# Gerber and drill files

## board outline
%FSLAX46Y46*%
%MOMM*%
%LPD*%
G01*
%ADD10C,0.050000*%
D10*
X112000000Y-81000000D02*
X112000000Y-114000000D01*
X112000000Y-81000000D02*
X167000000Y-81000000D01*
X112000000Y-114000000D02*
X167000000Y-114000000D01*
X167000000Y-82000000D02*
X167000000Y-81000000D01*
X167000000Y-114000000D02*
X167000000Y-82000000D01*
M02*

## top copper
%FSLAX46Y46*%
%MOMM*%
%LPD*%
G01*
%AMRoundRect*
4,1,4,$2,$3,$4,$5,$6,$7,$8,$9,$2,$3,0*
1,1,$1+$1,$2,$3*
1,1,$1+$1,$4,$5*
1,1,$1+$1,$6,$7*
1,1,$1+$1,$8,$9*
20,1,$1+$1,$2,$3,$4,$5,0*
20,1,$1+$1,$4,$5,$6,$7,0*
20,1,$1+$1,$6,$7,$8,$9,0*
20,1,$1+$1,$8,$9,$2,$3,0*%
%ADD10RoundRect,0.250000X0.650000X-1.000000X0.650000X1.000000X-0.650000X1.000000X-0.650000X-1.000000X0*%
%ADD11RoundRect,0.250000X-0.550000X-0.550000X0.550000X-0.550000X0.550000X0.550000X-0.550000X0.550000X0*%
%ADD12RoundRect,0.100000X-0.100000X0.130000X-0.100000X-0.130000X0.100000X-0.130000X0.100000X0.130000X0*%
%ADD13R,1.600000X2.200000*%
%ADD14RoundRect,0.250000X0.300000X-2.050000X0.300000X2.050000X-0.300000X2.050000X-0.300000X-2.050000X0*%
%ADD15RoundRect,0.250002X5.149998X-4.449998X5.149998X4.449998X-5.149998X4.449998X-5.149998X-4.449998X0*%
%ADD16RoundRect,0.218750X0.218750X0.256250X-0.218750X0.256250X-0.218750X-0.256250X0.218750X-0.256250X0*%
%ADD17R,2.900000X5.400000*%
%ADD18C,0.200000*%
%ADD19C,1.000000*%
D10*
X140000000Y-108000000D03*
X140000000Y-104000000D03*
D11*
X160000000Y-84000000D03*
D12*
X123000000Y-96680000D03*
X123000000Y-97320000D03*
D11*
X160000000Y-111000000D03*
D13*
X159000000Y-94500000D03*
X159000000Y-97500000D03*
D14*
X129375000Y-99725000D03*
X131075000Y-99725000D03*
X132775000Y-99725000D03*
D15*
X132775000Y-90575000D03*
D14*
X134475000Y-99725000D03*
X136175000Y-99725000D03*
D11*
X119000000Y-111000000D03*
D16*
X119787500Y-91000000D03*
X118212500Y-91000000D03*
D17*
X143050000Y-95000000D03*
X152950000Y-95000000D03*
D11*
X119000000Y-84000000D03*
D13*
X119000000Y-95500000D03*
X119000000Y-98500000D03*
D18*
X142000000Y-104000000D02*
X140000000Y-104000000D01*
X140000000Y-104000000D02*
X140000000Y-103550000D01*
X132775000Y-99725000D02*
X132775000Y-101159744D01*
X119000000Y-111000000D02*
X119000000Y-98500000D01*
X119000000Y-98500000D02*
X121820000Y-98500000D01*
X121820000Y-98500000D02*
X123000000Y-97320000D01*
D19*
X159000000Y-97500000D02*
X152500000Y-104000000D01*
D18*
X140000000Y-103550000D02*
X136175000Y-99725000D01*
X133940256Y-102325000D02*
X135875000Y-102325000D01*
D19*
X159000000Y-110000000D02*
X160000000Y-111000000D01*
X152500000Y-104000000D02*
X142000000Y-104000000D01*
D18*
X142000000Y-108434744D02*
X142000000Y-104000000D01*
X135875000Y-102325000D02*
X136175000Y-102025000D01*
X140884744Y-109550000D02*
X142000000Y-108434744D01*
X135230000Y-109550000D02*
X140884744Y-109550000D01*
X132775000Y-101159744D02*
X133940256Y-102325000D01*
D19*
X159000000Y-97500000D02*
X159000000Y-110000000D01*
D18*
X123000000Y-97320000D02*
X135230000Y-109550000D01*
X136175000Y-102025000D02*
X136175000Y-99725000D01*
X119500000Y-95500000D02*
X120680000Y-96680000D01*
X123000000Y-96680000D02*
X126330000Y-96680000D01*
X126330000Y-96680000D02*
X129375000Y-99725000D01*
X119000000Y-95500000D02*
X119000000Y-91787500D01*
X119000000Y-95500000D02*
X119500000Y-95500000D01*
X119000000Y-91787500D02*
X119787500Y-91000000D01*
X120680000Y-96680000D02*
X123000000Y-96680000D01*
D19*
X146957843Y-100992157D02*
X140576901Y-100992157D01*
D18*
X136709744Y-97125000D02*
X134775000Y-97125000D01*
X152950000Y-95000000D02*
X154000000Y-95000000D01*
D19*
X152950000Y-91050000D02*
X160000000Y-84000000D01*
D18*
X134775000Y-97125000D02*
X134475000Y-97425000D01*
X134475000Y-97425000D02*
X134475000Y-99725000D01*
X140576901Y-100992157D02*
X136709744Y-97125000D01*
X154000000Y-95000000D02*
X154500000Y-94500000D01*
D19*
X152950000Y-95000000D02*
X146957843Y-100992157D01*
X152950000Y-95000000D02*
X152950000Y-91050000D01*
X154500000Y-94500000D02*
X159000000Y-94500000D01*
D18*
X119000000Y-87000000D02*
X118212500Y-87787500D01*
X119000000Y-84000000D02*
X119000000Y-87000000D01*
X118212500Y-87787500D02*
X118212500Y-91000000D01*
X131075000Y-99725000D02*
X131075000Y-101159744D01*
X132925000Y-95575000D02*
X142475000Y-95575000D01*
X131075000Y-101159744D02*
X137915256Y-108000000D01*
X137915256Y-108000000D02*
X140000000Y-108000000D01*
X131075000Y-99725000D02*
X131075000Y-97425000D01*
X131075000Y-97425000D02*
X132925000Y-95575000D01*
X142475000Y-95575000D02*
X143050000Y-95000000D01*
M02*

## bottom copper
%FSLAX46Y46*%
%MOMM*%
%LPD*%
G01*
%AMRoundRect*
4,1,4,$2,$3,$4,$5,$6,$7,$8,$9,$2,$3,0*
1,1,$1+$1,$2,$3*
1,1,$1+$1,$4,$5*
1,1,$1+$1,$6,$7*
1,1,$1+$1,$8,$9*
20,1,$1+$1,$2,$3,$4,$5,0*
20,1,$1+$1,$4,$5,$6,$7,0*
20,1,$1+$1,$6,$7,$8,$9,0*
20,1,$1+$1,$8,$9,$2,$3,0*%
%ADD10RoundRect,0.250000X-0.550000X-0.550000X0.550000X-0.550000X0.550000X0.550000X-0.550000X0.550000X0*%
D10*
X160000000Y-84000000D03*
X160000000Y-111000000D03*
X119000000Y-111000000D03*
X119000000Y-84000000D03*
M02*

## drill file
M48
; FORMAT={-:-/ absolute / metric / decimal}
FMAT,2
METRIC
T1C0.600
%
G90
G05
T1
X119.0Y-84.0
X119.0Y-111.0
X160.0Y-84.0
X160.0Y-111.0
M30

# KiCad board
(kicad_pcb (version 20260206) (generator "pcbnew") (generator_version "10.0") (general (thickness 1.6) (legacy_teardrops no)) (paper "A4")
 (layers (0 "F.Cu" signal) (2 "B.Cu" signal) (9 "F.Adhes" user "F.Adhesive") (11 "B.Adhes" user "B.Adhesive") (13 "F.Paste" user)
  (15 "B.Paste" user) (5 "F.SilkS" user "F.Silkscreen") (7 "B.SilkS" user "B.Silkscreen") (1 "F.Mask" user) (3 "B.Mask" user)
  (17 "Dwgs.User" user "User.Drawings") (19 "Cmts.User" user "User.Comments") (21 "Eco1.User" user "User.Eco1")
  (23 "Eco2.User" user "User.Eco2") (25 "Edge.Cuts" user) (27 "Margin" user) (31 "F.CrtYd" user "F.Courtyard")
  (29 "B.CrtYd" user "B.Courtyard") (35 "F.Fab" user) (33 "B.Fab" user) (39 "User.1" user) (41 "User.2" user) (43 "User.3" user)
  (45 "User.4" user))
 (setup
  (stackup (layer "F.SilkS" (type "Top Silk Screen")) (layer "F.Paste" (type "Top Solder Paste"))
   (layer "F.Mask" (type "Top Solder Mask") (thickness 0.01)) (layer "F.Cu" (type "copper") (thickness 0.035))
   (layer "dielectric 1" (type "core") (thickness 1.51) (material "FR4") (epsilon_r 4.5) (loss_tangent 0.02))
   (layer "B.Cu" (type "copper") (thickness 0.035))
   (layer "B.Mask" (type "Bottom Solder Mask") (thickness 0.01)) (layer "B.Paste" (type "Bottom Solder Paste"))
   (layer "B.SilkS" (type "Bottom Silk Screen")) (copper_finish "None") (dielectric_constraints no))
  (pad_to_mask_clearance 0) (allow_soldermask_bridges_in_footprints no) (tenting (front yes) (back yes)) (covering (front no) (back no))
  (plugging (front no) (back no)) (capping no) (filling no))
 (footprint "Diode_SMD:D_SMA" (layer "F.Cu") (at 140 106 90)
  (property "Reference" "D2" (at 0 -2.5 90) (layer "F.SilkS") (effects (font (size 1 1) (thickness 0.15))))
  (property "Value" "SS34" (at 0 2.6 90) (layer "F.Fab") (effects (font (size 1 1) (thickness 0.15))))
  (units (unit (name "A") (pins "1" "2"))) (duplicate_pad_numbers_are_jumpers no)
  (pad "1" smd roundrect (at -2 0 90) (size 2.5 1.8) (layers "F.Cu" "F.Mask" "F.Paste") (roundrect_rratio 0.1388888889) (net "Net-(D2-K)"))
  (pad "2" smd roundrect (at 2 0 90) (size 2.5 1.8) (layers "F.Cu" "F.Mask" "F.Paste") (roundrect_rratio 0.1388888889) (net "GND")))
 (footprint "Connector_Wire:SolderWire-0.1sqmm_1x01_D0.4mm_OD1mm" (layer "F.Cu") (at 160 84)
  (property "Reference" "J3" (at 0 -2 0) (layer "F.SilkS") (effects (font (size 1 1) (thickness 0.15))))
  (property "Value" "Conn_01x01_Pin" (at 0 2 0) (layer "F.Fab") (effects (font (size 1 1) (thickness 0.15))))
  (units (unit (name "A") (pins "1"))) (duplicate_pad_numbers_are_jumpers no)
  (pad "1" thru_hole roundrect (at 0 0) (size 1.6 1.6) (drill 0.6) (layers "*.Cu" "*.Mask") (remove_unused_layers no)
   (roundrect_rratio 0.15625) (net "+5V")))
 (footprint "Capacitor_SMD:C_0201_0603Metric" (layer "F.Cu") (at 123 97 -90)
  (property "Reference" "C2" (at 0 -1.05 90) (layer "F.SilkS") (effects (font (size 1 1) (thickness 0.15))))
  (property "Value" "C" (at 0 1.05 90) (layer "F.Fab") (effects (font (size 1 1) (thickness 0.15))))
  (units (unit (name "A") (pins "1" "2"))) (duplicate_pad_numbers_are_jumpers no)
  (pad "" smd roundrect (at -0.345 0 270) (size 0.318 0.36) (layers "F.Paste") (roundrect_rratio 0.25))
  (pad "" smd roundrect (at 0.345 0 270) (size 0.318 0.36) (layers "F.Paste") (roundrect_rratio 0.25))
  (pad "1" smd roundrect (at -0.32 0 270) (size 0.46 0.4) (layers "F.Cu" "F.Mask") (roundrect_rratio 0.25) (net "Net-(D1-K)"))
  (pad "2" smd roundrect (at 0.32 0 270) (size 0.46 0.4) (layers "F.Cu" "F.Mask") (roundrect_rratio 0.25) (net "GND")))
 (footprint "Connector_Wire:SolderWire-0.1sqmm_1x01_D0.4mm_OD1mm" (layer "F.Cu") (at 160 111)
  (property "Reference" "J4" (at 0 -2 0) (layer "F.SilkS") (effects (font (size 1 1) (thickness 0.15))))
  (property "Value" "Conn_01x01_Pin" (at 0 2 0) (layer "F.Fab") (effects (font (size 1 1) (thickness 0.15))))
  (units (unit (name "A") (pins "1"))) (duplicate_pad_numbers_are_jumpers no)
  (pad "1" thru_hole roundrect (at 0 0) (size 1.6 1.6) (drill 0.6) (layers "*.Cu" "*.Mask") (remove_unused_layers no)
   (roundrect_rratio 0.15625) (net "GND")))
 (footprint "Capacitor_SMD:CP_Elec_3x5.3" (layer "F.Cu") (at 159 96 -90)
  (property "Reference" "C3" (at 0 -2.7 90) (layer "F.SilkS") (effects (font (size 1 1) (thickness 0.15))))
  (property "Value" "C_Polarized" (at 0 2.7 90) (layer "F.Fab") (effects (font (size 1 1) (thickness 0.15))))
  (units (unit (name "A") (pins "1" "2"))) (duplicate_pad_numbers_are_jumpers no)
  (pad "1" smd rect (at -1.5 0 270) (size 2.2 1.6) (layers "F.Cu" "F.Mask" "F.Paste") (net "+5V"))
  (pad "2" smd rect (at 1.5 0 270) (size 2.2 1.6) (layers "F.Cu" "F.Mask" "F.Paste") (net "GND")))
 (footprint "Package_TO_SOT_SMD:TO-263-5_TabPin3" (layer "F.Cu") (at 132.775 92.075 90)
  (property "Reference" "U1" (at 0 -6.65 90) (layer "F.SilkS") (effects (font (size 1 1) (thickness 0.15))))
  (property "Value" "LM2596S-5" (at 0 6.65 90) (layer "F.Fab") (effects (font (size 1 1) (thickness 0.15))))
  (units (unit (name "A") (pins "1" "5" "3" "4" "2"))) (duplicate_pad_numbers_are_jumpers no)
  (pad "" smd roundrect (at -0.925 -2.775 90) (size 4.55 5.25) (layers "F.Paste") (roundrect_rratio 0.054945))
  (pad "" smd roundrect (at -0.925 2.775 90) (size 4.55 5.25) (layers "F.Paste") (roundrect_rratio 0.054945))
  (pad "" smd roundrect (at 3.925 -2.775 90) (size 4.55 5.25) (layers "F.Paste") (roundrect_rratio 0.054945))
  (pad "" smd roundrect (at 3.925 2.775 90) (size 4.55 5.25) (layers "F.Paste") (roundrect_rratio 0.054945))
  (pad "1" smd roundrect (at -7.65 -3.4 90) (size 4.6 1.1) (layers "F.Cu" "F.Mask" "F.Paste") (roundrect_rratio 0.227273) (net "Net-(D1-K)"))
  (pad "2" smd roundrect (at -7.65 -1.7 90) (size 4.6 1.1) (layers "F.Cu" "F.Mask" "F.Paste") (roundrect_rratio 0.227273) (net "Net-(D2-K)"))
  (pad "3" smd roundrect (at -7.65 0 90) (size 4.6 1.1) (layers "F.Cu" "F.Mask" "F.Paste") (roundrect_rratio 0.227273) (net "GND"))
  (pad "3" smd roundrect (at 1.5 0 90) (size 9.4 10.8) (layers "F.Cu" "F.Mask") (roundrect_rratio 0.026596) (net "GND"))
  (pad "4" smd roundrect (at -7.65 1.7 90) (size 4.6 1.1) (layers "F.Cu" "F.Mask" "F.Paste") (roundrect_rratio 0.227273) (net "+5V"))
  (pad "5" smd roundrect (at -7.65 3.4 90) (size 4.6 1.1) (layers "F.Cu" "F.Mask" "F.Paste") (roundrect_rratio 0.227273) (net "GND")))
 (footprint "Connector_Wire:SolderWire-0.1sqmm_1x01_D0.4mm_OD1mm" (layer "F.Cu") (at 119 111)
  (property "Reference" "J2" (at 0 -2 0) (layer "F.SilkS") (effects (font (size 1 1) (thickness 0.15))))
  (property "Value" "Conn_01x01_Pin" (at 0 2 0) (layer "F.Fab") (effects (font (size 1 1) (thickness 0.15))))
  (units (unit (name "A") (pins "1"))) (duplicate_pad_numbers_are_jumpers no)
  (pad "1" thru_hole roundrect (at 0 0) (size 1.6 1.6) (drill 0.6) (layers "*.Cu" "*.Mask") (remove_unused_layers no)
   (roundrect_rratio 0.15625) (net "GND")))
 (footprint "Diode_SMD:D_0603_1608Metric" (layer "F.Cu") (at 119 91 180)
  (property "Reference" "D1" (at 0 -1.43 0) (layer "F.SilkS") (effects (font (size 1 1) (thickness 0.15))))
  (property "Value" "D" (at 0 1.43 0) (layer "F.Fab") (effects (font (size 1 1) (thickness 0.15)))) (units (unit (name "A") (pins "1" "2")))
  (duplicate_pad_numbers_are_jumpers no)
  (pad "1" smd roundrect (at -0.7875 0 180) (size 0.875 0.95) (layers "F.Cu" "F.Mask" "F.Paste") (roundrect_rratio 0.25) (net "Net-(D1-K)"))
  (pad "2" smd roundrect (at 0.7875 0 180) (size 0.875 0.95) (layers "F.Cu" "F.Mask" "F.Paste") (roundrect_rratio 0.25) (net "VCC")))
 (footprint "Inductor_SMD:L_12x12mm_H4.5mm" (layer "F.Cu") (at 148 95)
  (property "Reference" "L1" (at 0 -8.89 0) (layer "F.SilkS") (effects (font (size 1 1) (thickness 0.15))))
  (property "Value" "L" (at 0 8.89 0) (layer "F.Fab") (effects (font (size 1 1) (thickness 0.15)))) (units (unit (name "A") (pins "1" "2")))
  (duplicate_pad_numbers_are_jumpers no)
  (pad "1" smd rect (at -4.95 0) (size 2.9 5.4) (layers "F.Cu" "F.Mask" "F.Paste") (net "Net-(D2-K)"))
  (pad "2" smd rect (at 4.95 0) (size 2.9 5.4) (layers "F.Cu" "F.Mask" "F.Paste") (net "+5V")))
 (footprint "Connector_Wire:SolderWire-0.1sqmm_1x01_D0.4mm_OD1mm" (layer "F.Cu") (at 119 84)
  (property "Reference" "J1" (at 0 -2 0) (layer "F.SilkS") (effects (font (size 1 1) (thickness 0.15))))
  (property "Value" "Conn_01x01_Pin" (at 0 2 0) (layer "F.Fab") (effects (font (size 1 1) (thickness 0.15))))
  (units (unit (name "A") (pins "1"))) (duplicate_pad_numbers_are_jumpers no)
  (pad "1" thru_hole roundrect (at 0 0) (size 1.6 1.6) (drill 0.6) (layers "*.Cu" "*.Mask") (remove_unused_layers no)
   (roundrect_rratio 0.15625) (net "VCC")))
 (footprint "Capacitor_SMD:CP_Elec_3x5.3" (layer "F.Cu") (at 119 97 -90)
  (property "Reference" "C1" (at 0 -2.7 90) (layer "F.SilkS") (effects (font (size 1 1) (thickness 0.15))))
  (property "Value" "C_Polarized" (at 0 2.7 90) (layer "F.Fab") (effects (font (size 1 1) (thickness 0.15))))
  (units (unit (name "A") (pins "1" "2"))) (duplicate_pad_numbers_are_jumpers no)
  (pad "1" smd rect (at -1.5 0 270) (size 2.2 1.6) (layers "F.Cu" "F.Mask" "F.Paste") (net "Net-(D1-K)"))
  (pad "2" smd rect (at 1.5 0 270) (size 2.2 1.6) (layers "F.Cu" "F.Mask" "F.Paste") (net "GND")))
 (gr_line (start 112 81) (end 112 114) (stroke (width 0.05) (type default)) (layer "Edge.Cuts"))
 (gr_line (start 112 81) (end 167 81) (stroke (width 0.05) (type default)) (layer "Edge.Cuts"))
 (gr_line (start 112 114) (end 167 114) (stroke (width 0.05) (type default)) (layer "Edge.Cuts"))
 (gr_line (start 167 82) (end 167 81) (stroke (width 0.05) (type default)) (layer "Edge.Cuts"))
 (gr_line (start 167 114) (end 167 82) (stroke (width 0.05) (type default)) (layer "Edge.Cuts"))
 (segment (start 142 104) (end 140 104) (width 0.2) (layer "F.Cu") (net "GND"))
 (segment (start 140 104) (end 140 103.55) (width 0.2) (layer "F.Cu") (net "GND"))
 (segment (start 132.775 99.725) (end 132.775 101.159744) (width 0.2) (layer "F.Cu") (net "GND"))
 (segment (start 119 111) (end 119 98.5) (width 0.2) (layer "F.Cu") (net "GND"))
 (segment (start 119 98.5) (end 121.82 98.5) (width 0.2) (layer "F.Cu") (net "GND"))
 (segment (start 121.82 98.5) (end 123 97.32) (width 0.2) (layer "F.Cu") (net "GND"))
 (segment (start 159 97.5) (end 152.5 104) (width 1) (layer "F.Cu") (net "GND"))
 (segment (start 140 103.55) (end 136.175 99.725) (width 0.2) (layer "F.Cu") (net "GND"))
 (segment (start 133.940256 102.325) (end 135.875 102.325) (width 0.2) (layer "F.Cu") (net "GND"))
 (segment (start 159 110) (end 160 111) (width 1) (layer "F.Cu") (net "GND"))
 (segment (start 152.5 104) (end 142 104) (width 1) (layer "F.Cu") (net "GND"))
 (segment (start 142 108.434744) (end 142 104) (width 0.2) (layer "F.Cu") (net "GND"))
 (segment (start 135.875 102.325) (end 136.175 102.025) (width 0.2) (layer "F.Cu") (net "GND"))
 (segment (start 140.884744 109.55) (end 142 108.434744) (width 0.2) (layer "F.Cu") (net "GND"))
 (segment (start 135.23 109.55) (end 140.884744 109.55) (width 0.2) (layer "F.Cu") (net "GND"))
 (segment (start 132.775 101.159744) (end 133.940256 102.325) (width 0.2) (layer "F.Cu") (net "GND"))
 (segment (start 159 97.5) (end 159 110) (width 1) (layer "F.Cu") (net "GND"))
 (segment (start 123 97.32) (end 135.23 109.55) (width 0.2) (layer "F.Cu") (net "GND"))
 (segment (start 136.175 102.025) (end 136.175 99.725) (width 0.2) (layer "F.Cu") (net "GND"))
 (segment (start 119.5 95.5) (end 120.68 96.68) (width 0.2) (layer "F.Cu") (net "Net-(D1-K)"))
 (segment (start 123 96.68) (end 126.33 96.68) (width 0.2) (layer "F.Cu") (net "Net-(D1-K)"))
 (segment (start 126.33 96.68) (end 129.375 99.725) (width 0.2) (layer "F.Cu") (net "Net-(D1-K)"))
 (segment (start 119 95.5) (end 119 91.7875) (width 0.2) (layer "F.Cu") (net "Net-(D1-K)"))
 (segment (start 119 95.5) (end 119.5 95.5) (width 0.2) (layer "F.Cu") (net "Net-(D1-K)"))
 (segment (start 119 91.7875) (end 119.7875 91) (width 0.2) (layer "F.Cu") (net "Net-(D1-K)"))
 (segment (start 120.68 96.68) (end 123 96.68) (width 0.2) (layer "F.Cu") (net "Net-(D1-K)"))
 (segment (start 146.957843 100.992157) (end 140.576901 100.992157) (width 1) (layer "F.Cu") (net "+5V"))
 (segment (start 136.709744 97.125) (end 134.775 97.125) (width 0.2) (layer "F.Cu") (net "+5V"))
 (segment (start 152.95 95) (end 154 95) (width 0.2) (layer "F.Cu") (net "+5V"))
 (segment (start 152.95 91.05) (end 160 84) (width 1) (layer "F.Cu") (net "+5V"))
 (segment (start 134.775 97.125) (end 134.475 97.425) (width 0.2) (layer "F.Cu") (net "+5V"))
 (segment (start 134.475 97.425) (end 134.475 99.725) (width 0.2) (layer "F.Cu") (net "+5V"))
 (segment (start 140.576901 100.992157) (end 136.709744 97.125) (width 0.2) (layer "F.Cu") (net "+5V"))
 (segment (start 154 95) (end 154.5 94.5) (width 0.2) (layer "F.Cu") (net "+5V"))
 (segment (start 152.95 95) (end 146.957843 100.992157) (width 1) (layer "F.Cu") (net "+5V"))
 (segment (start 152.95 95) (end 152.95 91.05) (width 1) (layer "F.Cu") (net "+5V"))
 (segment (start 154.5 94.5) (end 159 94.5) (width 1) (layer "F.Cu") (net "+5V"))
 (segment (start 119 87) (end 118.2125 87.7875) (width 0.2) (layer "F.Cu") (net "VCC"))
 (segment (start 119 84) (end 119 87) (width 0.2) (layer "F.Cu") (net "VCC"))
 (segment (start 118.2125 87.7875) (end 118.2125 91) (width 0.2) (layer "F.Cu") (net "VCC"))
 (segment (start 131.075 99.725) (end 131.075 101.159744) (width 0.2) (layer "F.Cu") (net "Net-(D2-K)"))
 (segment (start 132.925 95.575) (end 142.475 95.575) (width 0.2) (layer "F.Cu") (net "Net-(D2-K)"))
 (segment (start 131.075 101.159744) (end 137.915256 108) (width 0.2) (layer "F.Cu") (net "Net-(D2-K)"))
 (segment (start 137.915256 108) (end 140 108) (width 0.2) (layer "F.Cu") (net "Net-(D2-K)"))
 (segment (start 131.075 99.725) (end 131.075 97.425) (width 0.2) (layer "F.Cu") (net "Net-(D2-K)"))
 (segment (start 131.075 97.425) (end 132.925 95.575) (width 0.2) (layer "F.Cu") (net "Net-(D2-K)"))
 (segment (start 142.475 95.575) (end 143.05 95) (width 0.2) (layer "F.Cu") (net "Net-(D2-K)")))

